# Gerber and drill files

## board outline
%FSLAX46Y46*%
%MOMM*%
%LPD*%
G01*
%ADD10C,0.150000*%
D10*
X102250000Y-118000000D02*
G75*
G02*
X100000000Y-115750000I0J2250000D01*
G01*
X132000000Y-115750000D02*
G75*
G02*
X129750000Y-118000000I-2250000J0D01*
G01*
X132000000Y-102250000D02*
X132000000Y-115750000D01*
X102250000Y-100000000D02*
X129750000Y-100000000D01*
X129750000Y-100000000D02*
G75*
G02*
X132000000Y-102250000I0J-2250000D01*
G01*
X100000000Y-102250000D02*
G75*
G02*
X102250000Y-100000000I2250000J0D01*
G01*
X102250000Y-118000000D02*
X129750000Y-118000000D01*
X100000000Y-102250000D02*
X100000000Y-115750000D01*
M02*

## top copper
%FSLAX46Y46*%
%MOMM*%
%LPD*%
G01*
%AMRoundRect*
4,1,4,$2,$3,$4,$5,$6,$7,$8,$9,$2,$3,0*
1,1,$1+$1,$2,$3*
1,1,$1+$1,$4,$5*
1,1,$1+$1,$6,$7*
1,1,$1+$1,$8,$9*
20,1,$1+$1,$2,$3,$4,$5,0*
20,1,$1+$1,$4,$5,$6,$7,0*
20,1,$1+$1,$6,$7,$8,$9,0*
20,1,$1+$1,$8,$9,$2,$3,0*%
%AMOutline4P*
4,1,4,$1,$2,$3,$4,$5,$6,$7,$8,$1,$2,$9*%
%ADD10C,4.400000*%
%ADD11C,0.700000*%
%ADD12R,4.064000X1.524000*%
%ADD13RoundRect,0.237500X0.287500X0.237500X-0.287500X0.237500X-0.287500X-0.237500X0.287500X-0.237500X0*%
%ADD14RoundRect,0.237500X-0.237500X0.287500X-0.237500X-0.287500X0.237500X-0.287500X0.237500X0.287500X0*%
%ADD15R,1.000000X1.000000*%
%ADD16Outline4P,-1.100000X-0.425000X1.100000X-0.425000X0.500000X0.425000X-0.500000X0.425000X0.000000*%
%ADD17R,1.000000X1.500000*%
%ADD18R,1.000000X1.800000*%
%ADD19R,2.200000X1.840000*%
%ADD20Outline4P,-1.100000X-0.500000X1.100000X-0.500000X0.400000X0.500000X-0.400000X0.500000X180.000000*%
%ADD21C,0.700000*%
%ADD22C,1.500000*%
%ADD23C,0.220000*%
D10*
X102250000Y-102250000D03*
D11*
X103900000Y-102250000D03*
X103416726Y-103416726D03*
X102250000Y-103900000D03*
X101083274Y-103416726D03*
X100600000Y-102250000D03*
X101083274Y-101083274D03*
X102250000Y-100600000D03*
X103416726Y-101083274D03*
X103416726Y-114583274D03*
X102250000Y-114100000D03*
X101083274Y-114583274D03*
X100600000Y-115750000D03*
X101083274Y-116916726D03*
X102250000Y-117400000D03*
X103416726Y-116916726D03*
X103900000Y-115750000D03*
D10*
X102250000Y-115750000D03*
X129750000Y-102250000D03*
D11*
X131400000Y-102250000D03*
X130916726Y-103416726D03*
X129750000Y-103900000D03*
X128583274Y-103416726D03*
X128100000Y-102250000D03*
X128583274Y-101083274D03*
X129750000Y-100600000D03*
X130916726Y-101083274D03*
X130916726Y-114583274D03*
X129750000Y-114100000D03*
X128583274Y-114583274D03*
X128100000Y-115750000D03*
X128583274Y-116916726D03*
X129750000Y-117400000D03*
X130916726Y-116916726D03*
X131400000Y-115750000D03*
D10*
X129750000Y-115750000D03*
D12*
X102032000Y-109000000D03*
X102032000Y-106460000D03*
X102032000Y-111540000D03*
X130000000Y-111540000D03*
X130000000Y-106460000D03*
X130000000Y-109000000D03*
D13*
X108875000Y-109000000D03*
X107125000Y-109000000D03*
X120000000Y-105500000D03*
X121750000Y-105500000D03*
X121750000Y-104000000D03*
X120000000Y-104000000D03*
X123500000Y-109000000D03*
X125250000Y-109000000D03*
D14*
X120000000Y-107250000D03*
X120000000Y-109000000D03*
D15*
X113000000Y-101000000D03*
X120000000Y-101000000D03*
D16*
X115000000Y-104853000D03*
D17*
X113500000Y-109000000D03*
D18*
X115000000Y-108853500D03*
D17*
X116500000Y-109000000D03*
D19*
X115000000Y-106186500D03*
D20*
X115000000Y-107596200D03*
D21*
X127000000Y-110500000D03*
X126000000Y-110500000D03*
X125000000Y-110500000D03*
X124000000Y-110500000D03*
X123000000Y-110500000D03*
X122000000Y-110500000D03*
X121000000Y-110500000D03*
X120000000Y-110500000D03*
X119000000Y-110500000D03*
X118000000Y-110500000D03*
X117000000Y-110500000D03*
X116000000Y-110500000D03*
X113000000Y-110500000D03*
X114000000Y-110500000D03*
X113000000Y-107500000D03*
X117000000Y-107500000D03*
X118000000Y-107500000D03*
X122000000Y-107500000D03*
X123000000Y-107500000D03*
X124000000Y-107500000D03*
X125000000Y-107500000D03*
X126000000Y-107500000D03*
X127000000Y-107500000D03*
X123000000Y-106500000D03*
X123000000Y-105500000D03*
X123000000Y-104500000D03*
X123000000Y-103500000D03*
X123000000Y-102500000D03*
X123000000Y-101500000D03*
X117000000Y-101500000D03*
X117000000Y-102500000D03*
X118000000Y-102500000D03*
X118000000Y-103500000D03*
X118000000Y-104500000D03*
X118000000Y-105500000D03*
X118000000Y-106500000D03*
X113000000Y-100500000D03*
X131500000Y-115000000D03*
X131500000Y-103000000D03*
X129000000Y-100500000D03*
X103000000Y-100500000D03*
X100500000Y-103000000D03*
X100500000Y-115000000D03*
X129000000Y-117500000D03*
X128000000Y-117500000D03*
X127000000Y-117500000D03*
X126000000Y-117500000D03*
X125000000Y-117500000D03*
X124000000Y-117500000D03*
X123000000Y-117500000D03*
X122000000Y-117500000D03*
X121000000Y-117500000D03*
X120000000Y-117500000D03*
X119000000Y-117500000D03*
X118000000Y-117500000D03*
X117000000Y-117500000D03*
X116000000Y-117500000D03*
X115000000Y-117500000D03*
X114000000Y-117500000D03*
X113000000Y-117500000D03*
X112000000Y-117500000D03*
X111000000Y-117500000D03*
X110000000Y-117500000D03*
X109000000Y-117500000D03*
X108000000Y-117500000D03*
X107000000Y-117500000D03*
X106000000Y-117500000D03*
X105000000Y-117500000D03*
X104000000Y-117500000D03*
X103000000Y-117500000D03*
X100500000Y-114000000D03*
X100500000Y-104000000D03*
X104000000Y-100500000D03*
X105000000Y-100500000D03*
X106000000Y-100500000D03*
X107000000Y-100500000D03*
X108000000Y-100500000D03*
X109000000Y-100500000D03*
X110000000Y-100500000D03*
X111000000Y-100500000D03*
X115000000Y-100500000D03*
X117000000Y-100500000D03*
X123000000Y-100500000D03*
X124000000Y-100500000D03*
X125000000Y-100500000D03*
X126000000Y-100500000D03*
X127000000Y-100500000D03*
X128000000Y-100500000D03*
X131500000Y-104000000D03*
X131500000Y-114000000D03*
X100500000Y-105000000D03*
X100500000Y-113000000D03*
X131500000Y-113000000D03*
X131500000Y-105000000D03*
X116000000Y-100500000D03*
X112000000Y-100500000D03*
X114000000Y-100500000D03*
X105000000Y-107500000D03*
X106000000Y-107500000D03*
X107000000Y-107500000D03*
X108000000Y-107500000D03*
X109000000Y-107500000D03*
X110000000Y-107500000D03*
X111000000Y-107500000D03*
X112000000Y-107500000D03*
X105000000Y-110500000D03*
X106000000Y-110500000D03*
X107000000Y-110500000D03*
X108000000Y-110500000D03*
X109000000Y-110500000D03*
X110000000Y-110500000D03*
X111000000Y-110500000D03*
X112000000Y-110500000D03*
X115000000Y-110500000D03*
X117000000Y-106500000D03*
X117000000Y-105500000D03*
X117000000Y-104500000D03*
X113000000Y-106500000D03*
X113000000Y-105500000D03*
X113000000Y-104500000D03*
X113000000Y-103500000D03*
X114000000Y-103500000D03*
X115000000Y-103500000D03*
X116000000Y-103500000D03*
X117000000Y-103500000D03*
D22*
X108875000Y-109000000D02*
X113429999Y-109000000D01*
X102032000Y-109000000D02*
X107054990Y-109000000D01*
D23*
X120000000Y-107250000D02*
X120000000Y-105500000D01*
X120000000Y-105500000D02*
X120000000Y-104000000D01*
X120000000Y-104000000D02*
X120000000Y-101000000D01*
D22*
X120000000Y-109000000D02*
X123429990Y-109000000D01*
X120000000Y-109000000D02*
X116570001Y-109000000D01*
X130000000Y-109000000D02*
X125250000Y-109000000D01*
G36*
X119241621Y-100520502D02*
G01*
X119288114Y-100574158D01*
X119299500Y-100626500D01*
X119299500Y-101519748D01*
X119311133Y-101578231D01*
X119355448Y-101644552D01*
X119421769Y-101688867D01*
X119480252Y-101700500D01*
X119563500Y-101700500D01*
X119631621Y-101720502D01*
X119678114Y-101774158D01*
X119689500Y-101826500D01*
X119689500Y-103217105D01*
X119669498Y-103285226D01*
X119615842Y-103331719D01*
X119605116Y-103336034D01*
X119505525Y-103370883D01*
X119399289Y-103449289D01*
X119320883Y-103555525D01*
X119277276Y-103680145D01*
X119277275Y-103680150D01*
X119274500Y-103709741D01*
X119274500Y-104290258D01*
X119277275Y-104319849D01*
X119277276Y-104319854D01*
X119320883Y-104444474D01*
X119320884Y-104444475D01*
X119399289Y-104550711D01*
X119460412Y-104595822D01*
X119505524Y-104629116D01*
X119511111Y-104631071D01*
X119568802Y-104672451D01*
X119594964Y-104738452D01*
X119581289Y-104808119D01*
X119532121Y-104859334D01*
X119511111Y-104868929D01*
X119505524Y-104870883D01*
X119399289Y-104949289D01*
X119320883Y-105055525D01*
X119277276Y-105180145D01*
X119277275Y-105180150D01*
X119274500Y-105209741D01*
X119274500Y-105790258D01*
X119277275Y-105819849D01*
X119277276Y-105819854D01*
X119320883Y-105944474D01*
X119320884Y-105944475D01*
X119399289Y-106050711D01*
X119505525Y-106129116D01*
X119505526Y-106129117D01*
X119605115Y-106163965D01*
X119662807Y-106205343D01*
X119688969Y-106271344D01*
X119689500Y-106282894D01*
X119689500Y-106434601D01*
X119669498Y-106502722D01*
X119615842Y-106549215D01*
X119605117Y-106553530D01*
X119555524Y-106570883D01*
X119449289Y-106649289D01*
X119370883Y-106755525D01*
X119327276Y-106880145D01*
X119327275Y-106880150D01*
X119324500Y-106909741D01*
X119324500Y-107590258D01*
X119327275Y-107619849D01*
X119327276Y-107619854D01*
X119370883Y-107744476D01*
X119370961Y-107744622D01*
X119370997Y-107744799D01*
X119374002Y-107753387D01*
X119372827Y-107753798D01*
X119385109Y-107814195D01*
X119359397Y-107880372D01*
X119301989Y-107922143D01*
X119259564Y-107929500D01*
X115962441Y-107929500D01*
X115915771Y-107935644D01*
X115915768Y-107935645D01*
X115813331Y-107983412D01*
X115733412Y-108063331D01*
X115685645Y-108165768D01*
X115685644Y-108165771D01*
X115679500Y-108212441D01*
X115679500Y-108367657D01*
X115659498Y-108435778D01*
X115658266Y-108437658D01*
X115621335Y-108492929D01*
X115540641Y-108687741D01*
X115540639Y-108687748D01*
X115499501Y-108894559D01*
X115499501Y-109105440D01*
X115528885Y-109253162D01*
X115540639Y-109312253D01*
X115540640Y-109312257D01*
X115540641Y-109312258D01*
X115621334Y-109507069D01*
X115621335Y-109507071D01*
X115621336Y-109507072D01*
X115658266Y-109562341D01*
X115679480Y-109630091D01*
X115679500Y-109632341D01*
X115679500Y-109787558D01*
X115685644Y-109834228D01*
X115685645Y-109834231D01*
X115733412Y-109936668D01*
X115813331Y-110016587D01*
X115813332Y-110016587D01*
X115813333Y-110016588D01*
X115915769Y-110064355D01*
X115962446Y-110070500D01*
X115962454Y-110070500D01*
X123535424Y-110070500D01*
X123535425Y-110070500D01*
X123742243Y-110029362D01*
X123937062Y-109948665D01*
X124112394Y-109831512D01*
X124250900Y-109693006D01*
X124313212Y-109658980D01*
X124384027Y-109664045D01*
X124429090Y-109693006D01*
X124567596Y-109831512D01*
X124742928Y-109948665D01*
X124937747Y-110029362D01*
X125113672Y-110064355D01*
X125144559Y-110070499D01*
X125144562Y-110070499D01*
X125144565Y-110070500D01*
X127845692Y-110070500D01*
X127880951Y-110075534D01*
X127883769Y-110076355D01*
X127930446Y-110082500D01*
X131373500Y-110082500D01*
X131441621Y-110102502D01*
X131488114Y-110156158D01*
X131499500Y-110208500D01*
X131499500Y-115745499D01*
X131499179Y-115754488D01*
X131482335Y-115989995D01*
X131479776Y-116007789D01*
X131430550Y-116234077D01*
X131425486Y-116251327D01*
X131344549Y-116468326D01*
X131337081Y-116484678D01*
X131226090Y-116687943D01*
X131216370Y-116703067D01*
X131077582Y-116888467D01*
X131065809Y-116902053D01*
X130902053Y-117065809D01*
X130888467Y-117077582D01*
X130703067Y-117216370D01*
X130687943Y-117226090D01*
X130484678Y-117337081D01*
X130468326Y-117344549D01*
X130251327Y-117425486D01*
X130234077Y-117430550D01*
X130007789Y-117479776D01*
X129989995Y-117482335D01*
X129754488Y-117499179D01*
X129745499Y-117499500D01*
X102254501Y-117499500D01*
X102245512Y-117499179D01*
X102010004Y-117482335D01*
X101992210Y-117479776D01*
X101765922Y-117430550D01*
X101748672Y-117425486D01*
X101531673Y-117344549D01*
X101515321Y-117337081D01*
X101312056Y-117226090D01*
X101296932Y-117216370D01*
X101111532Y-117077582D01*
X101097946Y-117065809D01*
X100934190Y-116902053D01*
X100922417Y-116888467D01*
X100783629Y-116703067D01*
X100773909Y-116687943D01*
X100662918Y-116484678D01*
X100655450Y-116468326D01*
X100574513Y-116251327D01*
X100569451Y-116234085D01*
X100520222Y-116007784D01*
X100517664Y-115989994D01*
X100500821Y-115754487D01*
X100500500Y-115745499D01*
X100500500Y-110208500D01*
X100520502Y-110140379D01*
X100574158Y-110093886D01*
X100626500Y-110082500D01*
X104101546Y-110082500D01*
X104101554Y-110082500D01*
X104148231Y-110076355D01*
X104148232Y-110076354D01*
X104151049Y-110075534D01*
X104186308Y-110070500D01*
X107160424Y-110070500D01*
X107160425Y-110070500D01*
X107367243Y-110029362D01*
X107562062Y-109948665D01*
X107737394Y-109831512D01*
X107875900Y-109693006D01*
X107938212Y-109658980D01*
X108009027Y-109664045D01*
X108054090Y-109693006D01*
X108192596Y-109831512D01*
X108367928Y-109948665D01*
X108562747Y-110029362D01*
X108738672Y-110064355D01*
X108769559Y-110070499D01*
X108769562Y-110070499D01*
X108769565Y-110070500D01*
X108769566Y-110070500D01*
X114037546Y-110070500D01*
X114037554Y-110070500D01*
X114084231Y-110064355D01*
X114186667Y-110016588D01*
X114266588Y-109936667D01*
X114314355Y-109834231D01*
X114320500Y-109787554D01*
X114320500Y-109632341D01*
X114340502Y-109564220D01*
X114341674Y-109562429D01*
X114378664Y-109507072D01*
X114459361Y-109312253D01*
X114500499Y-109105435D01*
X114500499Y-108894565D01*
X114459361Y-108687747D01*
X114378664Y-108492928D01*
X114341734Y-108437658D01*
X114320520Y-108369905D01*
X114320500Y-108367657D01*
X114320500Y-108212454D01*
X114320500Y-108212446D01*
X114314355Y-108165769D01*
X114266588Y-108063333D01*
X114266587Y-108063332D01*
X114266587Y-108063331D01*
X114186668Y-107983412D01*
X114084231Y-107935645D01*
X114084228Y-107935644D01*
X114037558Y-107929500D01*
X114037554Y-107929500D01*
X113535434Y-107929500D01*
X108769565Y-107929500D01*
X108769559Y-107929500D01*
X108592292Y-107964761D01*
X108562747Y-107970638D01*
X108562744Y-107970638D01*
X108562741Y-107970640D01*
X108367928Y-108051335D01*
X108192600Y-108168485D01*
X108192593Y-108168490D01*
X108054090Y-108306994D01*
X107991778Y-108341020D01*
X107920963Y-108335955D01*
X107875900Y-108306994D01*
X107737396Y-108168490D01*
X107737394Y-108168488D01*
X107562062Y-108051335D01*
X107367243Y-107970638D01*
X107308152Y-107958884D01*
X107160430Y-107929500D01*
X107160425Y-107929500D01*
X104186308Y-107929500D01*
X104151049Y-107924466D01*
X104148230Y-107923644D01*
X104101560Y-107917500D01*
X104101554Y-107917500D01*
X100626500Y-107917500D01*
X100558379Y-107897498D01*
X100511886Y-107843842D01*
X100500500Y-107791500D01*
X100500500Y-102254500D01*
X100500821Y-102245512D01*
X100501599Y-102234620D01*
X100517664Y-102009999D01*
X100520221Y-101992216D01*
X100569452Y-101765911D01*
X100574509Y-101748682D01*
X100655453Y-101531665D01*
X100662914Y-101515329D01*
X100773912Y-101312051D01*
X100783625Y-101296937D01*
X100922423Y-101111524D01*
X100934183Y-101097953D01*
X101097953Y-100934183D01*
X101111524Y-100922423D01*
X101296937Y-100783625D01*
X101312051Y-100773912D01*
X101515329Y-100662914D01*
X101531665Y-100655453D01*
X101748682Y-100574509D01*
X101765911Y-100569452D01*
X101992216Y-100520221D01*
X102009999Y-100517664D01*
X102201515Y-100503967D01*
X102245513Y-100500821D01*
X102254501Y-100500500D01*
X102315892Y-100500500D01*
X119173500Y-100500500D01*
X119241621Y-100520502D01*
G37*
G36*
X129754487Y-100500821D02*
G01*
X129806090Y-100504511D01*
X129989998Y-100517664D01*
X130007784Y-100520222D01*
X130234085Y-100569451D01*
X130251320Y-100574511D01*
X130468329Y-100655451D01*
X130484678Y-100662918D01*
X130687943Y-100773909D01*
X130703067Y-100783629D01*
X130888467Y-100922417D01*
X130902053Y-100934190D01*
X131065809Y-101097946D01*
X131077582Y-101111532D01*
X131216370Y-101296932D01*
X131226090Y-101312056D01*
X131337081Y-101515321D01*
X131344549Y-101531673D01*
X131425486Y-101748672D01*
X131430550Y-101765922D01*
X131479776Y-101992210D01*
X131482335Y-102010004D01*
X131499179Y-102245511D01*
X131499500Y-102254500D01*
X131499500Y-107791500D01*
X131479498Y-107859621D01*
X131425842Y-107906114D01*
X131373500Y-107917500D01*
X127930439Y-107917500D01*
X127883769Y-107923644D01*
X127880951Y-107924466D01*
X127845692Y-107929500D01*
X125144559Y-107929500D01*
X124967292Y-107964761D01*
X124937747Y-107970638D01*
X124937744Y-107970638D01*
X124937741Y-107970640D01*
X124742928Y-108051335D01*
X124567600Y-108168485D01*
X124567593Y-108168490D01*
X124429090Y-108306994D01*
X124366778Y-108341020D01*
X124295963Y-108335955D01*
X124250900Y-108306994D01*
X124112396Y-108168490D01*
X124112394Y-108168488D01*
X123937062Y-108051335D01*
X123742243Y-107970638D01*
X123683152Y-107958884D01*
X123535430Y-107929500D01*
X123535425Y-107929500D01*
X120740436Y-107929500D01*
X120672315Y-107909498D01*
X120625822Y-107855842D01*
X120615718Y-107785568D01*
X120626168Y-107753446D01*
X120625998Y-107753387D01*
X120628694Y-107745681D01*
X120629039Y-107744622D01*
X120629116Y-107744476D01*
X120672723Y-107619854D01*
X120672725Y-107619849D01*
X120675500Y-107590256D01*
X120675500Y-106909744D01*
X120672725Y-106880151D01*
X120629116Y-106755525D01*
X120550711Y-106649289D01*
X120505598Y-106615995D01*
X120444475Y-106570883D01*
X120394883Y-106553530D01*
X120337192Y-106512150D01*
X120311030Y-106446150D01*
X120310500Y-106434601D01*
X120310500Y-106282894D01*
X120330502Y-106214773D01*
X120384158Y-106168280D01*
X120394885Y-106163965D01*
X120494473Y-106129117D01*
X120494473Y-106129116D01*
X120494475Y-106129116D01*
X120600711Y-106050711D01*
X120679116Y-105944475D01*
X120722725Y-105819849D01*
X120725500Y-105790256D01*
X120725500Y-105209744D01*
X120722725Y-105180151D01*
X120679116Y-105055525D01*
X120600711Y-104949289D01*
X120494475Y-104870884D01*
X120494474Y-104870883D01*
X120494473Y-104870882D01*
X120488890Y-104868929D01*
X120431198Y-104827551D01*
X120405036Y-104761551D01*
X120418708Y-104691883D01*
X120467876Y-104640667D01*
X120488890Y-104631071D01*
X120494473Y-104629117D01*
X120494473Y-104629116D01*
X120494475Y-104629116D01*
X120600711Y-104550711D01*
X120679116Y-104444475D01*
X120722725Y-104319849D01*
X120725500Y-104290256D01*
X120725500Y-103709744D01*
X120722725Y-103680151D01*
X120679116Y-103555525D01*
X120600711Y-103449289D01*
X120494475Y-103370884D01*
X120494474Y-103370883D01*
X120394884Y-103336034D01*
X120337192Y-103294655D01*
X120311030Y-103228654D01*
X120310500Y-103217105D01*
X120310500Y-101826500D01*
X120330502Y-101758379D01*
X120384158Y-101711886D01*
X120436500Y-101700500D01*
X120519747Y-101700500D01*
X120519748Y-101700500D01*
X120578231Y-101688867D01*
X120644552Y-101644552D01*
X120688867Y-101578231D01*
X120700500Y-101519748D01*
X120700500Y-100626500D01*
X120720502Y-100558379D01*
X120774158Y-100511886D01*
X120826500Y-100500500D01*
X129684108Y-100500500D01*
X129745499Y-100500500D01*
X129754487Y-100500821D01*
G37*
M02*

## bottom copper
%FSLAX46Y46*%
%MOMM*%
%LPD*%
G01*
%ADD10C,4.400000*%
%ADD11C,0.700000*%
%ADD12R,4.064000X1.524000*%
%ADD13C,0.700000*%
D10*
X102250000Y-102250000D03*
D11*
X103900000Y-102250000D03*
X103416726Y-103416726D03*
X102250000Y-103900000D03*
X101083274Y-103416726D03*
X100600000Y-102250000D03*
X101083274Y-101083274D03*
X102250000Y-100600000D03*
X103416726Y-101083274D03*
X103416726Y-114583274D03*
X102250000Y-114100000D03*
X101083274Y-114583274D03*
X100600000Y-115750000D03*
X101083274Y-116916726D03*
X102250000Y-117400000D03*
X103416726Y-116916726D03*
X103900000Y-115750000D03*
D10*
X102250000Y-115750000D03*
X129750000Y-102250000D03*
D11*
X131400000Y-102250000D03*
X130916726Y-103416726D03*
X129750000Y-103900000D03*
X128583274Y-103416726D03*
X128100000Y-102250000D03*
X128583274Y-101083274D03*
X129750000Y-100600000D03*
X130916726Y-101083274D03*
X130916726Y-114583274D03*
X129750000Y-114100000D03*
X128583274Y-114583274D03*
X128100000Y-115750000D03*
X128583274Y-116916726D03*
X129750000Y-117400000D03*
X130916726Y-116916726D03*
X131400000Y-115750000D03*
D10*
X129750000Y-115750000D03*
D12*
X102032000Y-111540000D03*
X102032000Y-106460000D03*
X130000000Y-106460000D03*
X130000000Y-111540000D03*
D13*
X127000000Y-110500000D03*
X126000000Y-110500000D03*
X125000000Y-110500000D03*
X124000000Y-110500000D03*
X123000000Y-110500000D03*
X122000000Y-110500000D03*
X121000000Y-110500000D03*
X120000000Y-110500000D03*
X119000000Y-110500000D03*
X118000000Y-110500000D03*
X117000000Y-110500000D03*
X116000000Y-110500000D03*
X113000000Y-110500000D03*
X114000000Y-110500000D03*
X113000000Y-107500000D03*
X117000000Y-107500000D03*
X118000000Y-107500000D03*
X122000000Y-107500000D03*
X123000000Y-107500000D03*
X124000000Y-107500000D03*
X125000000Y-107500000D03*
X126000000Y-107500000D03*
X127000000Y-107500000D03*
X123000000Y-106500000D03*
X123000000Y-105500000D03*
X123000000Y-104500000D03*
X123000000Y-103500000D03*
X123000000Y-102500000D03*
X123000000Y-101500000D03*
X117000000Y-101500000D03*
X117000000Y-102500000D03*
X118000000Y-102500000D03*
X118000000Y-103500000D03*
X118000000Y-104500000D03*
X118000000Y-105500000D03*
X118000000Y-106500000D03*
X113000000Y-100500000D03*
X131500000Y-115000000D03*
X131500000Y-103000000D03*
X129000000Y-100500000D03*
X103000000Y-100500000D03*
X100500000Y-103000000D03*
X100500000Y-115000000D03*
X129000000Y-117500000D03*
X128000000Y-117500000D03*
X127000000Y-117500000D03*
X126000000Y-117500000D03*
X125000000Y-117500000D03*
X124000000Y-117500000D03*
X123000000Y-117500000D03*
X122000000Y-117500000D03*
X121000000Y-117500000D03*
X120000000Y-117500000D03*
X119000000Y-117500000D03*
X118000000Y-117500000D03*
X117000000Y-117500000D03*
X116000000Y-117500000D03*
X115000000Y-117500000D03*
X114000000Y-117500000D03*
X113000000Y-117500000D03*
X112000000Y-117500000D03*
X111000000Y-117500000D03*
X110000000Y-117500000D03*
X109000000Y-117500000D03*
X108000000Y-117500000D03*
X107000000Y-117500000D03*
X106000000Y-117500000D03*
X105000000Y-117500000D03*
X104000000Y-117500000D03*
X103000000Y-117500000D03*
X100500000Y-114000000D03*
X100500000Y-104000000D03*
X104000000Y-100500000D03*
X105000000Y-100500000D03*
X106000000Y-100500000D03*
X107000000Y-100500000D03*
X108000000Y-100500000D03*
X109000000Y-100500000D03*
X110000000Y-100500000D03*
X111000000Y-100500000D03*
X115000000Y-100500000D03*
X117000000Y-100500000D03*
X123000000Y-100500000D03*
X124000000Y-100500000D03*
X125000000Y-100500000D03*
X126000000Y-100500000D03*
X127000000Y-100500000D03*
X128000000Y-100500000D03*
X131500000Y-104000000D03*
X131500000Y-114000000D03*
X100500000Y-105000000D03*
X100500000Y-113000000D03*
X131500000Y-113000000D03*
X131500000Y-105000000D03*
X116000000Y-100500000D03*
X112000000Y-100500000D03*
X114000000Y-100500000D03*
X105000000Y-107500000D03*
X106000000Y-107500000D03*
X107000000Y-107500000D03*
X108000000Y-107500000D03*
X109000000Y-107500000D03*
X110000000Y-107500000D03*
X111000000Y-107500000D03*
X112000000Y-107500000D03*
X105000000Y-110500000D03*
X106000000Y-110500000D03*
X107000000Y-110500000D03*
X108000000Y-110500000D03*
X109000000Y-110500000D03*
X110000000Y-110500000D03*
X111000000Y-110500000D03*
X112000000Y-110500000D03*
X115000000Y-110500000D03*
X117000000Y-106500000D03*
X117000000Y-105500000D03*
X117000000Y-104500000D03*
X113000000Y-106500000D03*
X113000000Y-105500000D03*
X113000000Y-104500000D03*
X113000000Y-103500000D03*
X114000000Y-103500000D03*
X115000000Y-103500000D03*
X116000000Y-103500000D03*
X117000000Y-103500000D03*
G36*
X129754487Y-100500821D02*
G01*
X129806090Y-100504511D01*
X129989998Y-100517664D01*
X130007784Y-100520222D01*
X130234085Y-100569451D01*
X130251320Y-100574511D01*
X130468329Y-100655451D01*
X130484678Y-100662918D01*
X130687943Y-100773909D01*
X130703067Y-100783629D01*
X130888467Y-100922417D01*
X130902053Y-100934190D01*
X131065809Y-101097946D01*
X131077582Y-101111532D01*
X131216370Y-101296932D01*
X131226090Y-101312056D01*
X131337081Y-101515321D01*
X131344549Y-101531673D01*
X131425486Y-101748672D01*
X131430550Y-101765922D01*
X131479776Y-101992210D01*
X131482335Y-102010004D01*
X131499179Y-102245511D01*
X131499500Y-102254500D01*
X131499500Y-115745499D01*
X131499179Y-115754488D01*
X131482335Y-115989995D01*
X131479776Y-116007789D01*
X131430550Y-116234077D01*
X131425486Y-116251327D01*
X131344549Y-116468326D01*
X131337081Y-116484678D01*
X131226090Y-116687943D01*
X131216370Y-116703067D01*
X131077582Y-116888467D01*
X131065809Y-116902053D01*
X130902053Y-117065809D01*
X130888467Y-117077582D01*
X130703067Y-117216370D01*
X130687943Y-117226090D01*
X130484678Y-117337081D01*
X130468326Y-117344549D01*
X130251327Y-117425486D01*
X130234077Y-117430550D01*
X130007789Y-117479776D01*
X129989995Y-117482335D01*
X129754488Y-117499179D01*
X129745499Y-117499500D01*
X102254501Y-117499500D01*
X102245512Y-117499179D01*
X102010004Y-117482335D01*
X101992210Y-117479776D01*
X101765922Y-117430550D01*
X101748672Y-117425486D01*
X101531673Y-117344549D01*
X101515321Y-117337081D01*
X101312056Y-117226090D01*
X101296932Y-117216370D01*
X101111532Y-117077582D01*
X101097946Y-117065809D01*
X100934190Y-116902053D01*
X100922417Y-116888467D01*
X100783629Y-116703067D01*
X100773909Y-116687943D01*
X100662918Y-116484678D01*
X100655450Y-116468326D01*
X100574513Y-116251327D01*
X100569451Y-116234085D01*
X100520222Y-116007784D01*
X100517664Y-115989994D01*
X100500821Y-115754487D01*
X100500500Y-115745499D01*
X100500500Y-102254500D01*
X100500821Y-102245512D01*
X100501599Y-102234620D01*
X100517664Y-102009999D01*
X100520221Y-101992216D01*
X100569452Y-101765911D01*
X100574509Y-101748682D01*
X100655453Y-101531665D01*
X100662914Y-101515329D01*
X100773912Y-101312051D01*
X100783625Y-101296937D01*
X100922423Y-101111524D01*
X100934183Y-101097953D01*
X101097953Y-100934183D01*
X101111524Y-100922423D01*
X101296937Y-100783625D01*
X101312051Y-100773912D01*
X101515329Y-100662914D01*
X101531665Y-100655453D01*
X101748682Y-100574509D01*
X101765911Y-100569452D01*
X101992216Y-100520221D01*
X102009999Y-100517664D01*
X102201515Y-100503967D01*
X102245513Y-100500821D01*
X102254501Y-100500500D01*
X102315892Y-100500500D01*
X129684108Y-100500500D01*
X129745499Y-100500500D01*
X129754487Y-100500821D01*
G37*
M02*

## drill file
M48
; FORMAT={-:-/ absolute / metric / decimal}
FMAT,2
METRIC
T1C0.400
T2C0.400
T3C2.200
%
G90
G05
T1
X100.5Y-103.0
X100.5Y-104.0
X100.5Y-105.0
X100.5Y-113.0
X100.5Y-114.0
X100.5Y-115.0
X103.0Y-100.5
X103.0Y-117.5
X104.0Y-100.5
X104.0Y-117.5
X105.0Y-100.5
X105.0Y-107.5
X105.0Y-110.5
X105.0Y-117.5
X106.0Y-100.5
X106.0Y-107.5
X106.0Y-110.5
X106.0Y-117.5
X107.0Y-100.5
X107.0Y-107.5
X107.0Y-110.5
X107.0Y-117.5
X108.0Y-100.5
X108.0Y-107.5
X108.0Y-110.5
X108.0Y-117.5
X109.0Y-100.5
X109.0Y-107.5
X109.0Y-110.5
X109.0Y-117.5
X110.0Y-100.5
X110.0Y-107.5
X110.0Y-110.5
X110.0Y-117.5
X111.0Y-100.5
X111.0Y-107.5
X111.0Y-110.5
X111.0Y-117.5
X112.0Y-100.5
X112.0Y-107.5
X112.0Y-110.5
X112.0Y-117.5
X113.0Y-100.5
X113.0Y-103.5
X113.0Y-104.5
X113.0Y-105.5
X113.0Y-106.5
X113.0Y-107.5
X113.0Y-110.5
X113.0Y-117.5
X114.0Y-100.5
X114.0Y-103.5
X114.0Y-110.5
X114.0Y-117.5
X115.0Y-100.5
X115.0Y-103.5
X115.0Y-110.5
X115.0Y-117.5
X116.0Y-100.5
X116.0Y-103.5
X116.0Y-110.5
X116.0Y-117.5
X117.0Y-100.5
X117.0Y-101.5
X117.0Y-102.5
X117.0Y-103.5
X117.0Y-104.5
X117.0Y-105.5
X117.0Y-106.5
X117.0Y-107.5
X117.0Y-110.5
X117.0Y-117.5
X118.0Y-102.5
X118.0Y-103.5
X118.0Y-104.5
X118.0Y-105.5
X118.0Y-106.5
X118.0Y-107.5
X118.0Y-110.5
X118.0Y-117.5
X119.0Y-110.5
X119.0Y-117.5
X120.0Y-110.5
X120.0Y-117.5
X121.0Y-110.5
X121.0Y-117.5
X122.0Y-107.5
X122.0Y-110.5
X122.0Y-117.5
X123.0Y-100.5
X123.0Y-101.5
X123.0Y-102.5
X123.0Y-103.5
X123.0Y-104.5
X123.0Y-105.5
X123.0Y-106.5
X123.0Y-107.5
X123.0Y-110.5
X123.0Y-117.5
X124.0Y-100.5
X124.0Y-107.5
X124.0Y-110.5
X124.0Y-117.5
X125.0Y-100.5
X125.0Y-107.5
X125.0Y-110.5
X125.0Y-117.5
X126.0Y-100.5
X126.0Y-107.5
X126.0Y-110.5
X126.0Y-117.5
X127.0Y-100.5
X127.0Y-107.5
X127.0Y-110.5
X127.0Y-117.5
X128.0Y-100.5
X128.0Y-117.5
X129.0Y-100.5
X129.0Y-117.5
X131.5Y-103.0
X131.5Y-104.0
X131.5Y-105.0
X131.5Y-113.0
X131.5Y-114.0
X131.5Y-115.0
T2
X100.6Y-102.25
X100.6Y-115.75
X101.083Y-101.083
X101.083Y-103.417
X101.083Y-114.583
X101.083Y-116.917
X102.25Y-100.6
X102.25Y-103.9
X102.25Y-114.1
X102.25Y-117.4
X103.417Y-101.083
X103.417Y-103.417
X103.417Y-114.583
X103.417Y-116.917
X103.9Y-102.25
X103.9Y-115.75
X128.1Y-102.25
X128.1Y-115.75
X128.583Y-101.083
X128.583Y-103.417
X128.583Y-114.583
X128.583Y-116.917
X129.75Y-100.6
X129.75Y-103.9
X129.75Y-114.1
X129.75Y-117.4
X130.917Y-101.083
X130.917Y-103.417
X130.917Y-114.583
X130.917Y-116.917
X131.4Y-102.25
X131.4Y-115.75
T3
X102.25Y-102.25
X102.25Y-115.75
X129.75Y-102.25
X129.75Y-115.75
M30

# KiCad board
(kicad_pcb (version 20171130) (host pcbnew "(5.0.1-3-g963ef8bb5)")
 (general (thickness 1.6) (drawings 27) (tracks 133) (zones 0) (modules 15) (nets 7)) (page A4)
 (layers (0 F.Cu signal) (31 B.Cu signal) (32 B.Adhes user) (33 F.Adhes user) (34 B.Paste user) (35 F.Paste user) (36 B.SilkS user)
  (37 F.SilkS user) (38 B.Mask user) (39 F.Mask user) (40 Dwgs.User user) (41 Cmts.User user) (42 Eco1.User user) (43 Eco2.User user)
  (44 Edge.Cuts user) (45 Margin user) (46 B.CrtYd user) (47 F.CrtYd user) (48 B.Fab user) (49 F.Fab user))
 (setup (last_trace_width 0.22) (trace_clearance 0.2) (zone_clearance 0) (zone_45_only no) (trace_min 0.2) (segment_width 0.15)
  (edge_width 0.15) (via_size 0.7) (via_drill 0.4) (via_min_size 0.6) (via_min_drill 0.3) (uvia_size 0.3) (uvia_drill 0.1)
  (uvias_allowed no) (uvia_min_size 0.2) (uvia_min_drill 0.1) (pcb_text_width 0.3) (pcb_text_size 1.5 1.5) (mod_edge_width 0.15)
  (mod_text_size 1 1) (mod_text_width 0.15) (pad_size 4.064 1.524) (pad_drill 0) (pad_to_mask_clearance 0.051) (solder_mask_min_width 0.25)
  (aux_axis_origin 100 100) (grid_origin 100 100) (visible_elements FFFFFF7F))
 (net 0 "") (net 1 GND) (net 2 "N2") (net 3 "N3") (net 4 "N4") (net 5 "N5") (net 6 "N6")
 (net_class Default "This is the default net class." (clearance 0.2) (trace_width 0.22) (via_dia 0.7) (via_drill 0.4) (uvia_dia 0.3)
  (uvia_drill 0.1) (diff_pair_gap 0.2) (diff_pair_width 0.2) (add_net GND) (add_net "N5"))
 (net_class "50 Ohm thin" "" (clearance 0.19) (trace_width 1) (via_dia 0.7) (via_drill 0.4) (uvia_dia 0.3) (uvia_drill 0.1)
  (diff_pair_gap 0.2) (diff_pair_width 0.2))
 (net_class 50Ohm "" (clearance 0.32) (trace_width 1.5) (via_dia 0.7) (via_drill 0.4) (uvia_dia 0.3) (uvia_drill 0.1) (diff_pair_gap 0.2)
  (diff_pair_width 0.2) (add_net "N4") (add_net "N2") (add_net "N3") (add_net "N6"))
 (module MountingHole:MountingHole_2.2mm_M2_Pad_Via (layer F.Cu) (at 102.25 102.25)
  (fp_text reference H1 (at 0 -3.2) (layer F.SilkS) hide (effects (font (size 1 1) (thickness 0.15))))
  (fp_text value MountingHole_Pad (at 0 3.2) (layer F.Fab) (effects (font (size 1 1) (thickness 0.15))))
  (pad 1 thru_hole circle (at 0 0) (size 4.4 4.4) (drill 2.2) (layers *.Cu *.Mask) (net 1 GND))
  (pad 1 thru_hole circle (at 1.65 0) (size 0.7 0.7) (drill 0.4) (layers *.Cu *.Mask) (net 1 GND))
  (pad 1 thru_hole circle (at 1.166726 1.166726) (size 0.7 0.7) (drill 0.4) (layers *.Cu *.Mask) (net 1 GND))
  (pad 1 thru_hole circle (at 0 1.65) (size 0.7 0.7) (drill 0.4) (layers *.Cu *.Mask) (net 1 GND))
  (pad 1 thru_hole circle (at -1.166726 1.166726) (size 0.7 0.7) (drill 0.4) (layers *.Cu *.Mask) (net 1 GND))
  (pad 1 thru_hole circle (at -1.65 0) (size 0.7 0.7) (drill 0.4) (layers *.Cu *.Mask) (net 1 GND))
  (pad 1 thru_hole circle (at -1.166726 -1.166726) (size 0.7 0.7) (drill 0.4) (layers *.Cu *.Mask) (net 1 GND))
  (pad 1 thru_hole circle (at 0 -1.65) (size 0.7 0.7) (drill 0.4) (layers *.Cu *.Mask) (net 1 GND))
  (pad 1 thru_hole circle (at 1.166726 -1.166726) (size 0.7 0.7) (drill 0.4) (layers *.Cu *.Mask) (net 1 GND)))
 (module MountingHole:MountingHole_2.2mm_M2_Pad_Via (layer F.Cu) (at 102.25 115.75)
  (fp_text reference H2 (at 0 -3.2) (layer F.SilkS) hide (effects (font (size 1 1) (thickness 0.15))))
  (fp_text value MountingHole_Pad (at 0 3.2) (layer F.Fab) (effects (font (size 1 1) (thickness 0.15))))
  (pad 1 thru_hole circle (at 1.166726 -1.166726) (size 0.7 0.7) (drill 0.4) (layers *.Cu *.Mask) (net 1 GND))
  (pad 1 thru_hole circle (at 0 -1.65) (size 0.7 0.7) (drill 0.4) (layers *.Cu *.Mask) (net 1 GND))
  (pad 1 thru_hole circle (at -1.166726 -1.166726) (size 0.7 0.7) (drill 0.4) (layers *.Cu *.Mask) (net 1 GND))
  (pad 1 thru_hole circle (at -1.65 0) (size 0.7 0.7) (drill 0.4) (layers *.Cu *.Mask) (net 1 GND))
  (pad 1 thru_hole circle (at -1.166726 1.166726) (size 0.7 0.7) (drill 0.4) (layers *.Cu *.Mask) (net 1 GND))
  (pad 1 thru_hole circle (at 0 1.65) (size 0.7 0.7) (drill 0.4) (layers *.Cu *.Mask) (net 1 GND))
  (pad 1 thru_hole circle (at 1.166726 1.166726) (size 0.7 0.7) (drill 0.4) (layers *.Cu *.Mask) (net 1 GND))
  (pad 1 thru_hole circle (at 1.65 0) (size 0.7 0.7) (drill 0.4) (layers *.Cu *.Mask) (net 1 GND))
  (pad 1 thru_hole circle (at 0 0) (size 4.4 4.4) (drill 2.2) (layers *.Cu *.Mask) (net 1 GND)))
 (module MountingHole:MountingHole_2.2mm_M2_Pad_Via (layer F.Cu) (at 129.75 102.25)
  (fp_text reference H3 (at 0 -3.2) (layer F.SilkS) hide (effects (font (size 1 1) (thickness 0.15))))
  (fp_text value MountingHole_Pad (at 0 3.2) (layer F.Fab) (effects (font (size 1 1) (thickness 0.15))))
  (pad 1 thru_hole circle (at 0 0) (size 4.4 4.4) (drill 2.2) (layers *.Cu *.Mask) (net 1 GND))
  (pad 1 thru_hole circle (at 1.65 0) (size 0.7 0.7) (drill 0.4) (layers *.Cu *.Mask) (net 1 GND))
  (pad 1 thru_hole circle (at 1.166726 1.166726) (size 0.7 0.7) (drill 0.4) (layers *.Cu *.Mask) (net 1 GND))
  (pad 1 thru_hole circle (at 0 1.65) (size 0.7 0.7) (drill 0.4) (layers *.Cu *.Mask) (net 1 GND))
  (pad 1 thru_hole circle (at -1.166726 1.166726) (size 0.7 0.7) (drill 0.4) (layers *.Cu *.Mask) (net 1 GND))
  (pad 1 thru_hole circle (at -1.65 0) (size 0.7 0.7) (drill 0.4) (layers *.Cu *.Mask) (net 1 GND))
  (pad 1 thru_hole circle (at -1.166726 -1.166726) (size 0.7 0.7) (drill 0.4) (layers *.Cu *.Mask) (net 1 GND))
  (pad 1 thru_hole circle (at 0 -1.65) (size 0.7 0.7) (drill 0.4) (layers *.Cu *.Mask) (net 1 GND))
  (pad 1 thru_hole circle (at 1.166726 -1.166726) (size 0.7 0.7) (drill 0.4) (layers *.Cu *.Mask) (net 1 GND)))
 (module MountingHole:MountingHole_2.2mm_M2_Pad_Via (layer F.Cu) (at 129.75 115.75)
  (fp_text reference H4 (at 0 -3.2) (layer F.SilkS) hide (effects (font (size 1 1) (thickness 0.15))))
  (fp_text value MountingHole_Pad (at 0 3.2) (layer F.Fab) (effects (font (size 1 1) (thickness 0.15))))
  (pad 1 thru_hole circle (at 1.166726 -1.166726) (size 0.7 0.7) (drill 0.4) (layers *.Cu *.Mask) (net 1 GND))
  (pad 1 thru_hole circle (at 0 -1.65) (size 0.7 0.7) (drill 0.4) (layers *.Cu *.Mask) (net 1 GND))
  (pad 1 thru_hole circle (at -1.166726 -1.166726) (size 0.7 0.7) (drill 0.4) (layers *.Cu *.Mask) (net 1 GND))
  (pad 1 thru_hole circle (at -1.65 0) (size 0.7 0.7) (drill 0.4) (layers *.Cu *.Mask) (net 1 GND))
  (pad 1 thru_hole circle (at -1.166726 1.166726) (size 0.7 0.7) (drill 0.4) (layers *.Cu *.Mask) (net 1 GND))
  (pad 1 thru_hole circle (at 0 1.65) (size 0.7 0.7) (drill 0.4) (layers *.Cu *.Mask) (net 1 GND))
  (pad 1 thru_hole circle (at 1.166726 1.166726) (size 0.7 0.7) (drill 0.4) (layers *.Cu *.Mask) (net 1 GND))
  (pad 1 thru_hole circle (at 1.65 0) (size 0.7 0.7) (drill 0.4) (layers *.Cu *.Mask) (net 1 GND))
  (pad 1 thru_hole circle (at 0 0) (size 4.4 4.4) (drill 2.2) (layers *.Cu *.Mask) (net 1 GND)))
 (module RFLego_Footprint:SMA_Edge (layer F.Cu) (at 100 109)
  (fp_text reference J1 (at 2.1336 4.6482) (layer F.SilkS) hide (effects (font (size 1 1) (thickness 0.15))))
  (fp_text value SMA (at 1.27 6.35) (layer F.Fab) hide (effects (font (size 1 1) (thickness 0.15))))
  (pad 1 smd rect (at 2.032 0) (size 4.064 1.524) (layers F.Cu F.Mask) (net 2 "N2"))
  (pad 2 smd rect (at 2.032 -2.54) (size 4.064 1.524) (layers F.Cu F.Mask) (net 1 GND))
  (pad 2 smd rect (at 2.032 2.54) (size 4.064 1.524) (layers B.Cu B.Mask) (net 1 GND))
  (pad 2 smd rect (at 2.032 -2.54) (size 4.064 1.524) (layers B.Cu B.Mask) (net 1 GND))
  (pad 2 smd rect (at 2.032 2.54) (size 4.064 1.524) (layers F.Cu F.Mask) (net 1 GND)))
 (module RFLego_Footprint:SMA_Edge (layer F.Cu) (at 127.968 109)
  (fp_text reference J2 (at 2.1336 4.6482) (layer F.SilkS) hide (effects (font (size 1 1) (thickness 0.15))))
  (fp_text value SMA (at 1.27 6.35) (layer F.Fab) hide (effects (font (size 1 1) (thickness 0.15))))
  (pad 2 smd rect (at 2.032 2.54) (size 4.064 1.524) (layers F.Cu F.Mask) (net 1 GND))
  (pad 2 smd rect (at 2.032 -2.54) (size 4.064 1.524) (layers B.Cu B.Mask) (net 1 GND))
  (pad 2 smd rect (at 2.032 2.54) (size 4.064 1.524) (layers B.Cu B.Mask) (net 1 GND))
  (pad 2 smd rect (at 2.032 -2.54) (size 4.064 1.524) (layers F.Cu F.Mask) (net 1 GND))
  (pad 1 smd rect (at 2.032 0) (size 4.064 1.524) (layers F.Cu F.Mask) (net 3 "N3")))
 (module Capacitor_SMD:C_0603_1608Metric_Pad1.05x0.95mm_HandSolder (layer F.Cu) (at 108 109 180)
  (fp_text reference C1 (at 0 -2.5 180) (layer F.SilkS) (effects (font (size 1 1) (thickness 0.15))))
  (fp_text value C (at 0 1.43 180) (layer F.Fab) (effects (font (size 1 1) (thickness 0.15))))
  (pad 1 smd roundrect (at -0.875 0 180) (size 1.05 0.95) (layers F.Cu F.Paste F.Mask) (roundrect_rratio 0.25) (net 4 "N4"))
  (pad 2 smd roundrect (at 0.875 0 180) (size 1.05 0.95) (layers F.Cu F.Paste F.Mask) (roundrect_rratio 0.25) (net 2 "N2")))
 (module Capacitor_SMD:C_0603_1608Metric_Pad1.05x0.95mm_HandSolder (layer F.Cu) (at 120.875 105.5 180)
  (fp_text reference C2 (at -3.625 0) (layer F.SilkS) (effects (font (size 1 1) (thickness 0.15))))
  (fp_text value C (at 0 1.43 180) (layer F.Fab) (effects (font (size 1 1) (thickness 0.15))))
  (pad 2 smd roundrect (at 0.875 0 180) (size 1.05 0.95) (layers F.Cu F.Paste F.Mask) (roundrect_rratio 0.25) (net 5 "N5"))
  (pad 1 smd roundrect (at -0.875 0 180) (size 1.05 0.95) (layers F.Cu F.Paste F.Mask) (roundrect_rratio 0.25) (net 1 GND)))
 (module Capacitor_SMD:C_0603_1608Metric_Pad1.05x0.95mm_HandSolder (layer F.Cu) (at 120.875 104 180)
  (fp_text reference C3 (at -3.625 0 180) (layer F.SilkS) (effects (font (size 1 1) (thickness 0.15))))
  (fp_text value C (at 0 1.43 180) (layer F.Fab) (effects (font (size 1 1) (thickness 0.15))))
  (pad 1 smd roundrect (at -0.875 0 180) (size 1.05 0.95) (layers F.Cu F.Paste F.Mask) (roundrect_rratio 0.25) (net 1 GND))
  (pad 2 smd roundrect (at 0.875 0 180) (size 1.05 0.95) (layers F.Cu F.Paste F.Mask) (roundrect_rratio 0.25) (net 5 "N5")))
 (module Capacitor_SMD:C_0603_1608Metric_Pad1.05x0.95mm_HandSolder (layer F.Cu) (at 124.375 109 180)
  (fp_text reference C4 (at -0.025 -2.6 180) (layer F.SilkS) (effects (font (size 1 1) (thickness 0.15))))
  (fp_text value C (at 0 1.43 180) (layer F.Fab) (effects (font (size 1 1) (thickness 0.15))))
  (pad 2 smd roundrect (at 0.875 0 180) (size 1.05 0.95) (layers F.Cu F.Paste F.Mask) (roundrect_rratio 0.25) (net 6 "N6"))
  (pad 1 smd roundrect (at -0.875 0 180) (size 1.05 0.95) (layers F.Cu F.Paste F.Mask) (roundrect_rratio 0.25) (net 3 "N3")))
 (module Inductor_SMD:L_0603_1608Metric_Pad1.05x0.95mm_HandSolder (layer F.Cu) (at 120 108.125 270)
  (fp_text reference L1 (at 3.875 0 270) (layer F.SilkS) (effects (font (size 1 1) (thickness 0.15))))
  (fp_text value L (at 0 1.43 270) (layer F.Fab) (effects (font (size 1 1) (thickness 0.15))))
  (pad 1 smd roundrect (at -0.875 0 270) (size 1.05 0.95) (layers F.Cu F.Paste F.Mask) (roundrect_rratio 0.25) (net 5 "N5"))
  (pad 2 smd roundrect (at 0.875 0 270) (size 1.05 0.95) (layers F.Cu F.Paste F.Mask) (roundrect_rratio 0.25) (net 6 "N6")))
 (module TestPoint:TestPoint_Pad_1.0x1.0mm (layer F.Cu) (at 113 101)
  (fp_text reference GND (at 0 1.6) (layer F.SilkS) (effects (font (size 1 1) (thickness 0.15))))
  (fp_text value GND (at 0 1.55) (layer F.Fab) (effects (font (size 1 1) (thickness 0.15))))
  (pad 1 smd rect (at 0 0) (size 1 1) (layers F.Cu F.Mask) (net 1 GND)))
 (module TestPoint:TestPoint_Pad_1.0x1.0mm (layer F.Cu) (at 120 101)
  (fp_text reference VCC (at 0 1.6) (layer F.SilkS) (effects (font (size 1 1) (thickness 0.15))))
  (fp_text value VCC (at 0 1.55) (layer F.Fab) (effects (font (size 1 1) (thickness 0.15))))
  (pad 1 smd rect (at 0 0) (size 1 1) (layers F.Cu F.Mask) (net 5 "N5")))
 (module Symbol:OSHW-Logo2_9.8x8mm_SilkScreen (layer B.Cu) (at 109.5 113 180)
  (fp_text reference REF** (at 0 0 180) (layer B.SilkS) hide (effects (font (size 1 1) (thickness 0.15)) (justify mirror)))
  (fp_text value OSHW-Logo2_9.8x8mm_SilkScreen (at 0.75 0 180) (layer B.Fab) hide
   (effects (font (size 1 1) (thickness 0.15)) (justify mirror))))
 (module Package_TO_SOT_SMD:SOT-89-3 (layer F.Cu) (at 115 107.52 90)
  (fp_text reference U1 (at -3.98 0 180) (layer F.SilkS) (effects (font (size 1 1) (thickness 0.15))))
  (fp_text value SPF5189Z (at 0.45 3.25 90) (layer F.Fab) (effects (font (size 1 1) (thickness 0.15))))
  (pad 2 smd trapezoid (at 2.667 0) (size 1.6 0.85) (rect_delta 0 0.6) (layers F.Cu F.Paste F.Mask) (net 1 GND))
  (pad 1 smd rect (at -1.48 -1.5) (size 1 1.5) (layers F.Cu F.Paste F.Mask) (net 4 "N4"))
  (pad 2 smd rect (at -1.3335 0) (size 1 1.8) (layers F.Cu F.Paste F.Mask) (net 1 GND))
  (pad 3 smd rect (at -1.48 1.5) (size 1 1.5) (layers F.Cu F.Paste F.Mask) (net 6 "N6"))
  (pad 2 smd rect (at 1.3335 0) (size 2.2 1.84) (layers F.Cu F.Paste F.Mask) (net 1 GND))
  (pad 2 smd trapezoid (at -0.0762 0 180) (size 1.5 1) (rect_delta 0 0.7) (layers F.Cu F.Paste F.Mask) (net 1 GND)))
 (gr_arc (start 102.25 115.75) (end 100 115.75) (angle -90) (layer Edge.Cuts) (width 0.15))
 (gr_arc (start 129.75 115.75) (end 129.75 118) (angle -90) (layer Edge.Cuts) (width 0.15))
 (gr_line (start 132 102.25) (end 132 115.75) (layer Edge.Cuts) (width 0.15))
 (gr_line (start 102.25 100) (end 129.75 100) (layer Edge.Cuts) (width 0.15))
 (gr_arc (start 129.75 102.25) (end 132 102.25) (angle -90) (layer Edge.Cuts) (width 0.15))
 (gr_arc (start 102.25 102.25) (end 102.25 100) (angle -90) (layer Edge.Cuts) (width 0.15))
 (gr_line (start 102.25 118) (end 129.75 118) (layer Edge.Cuts) (width 0.15))
 (gr_line (start 100 102.25) (end 100 115.75) (layer Edge.Cuts) (width 0.15))
 (via (at 127 110.5) (size 0.7) (drill 0.4) (layers F.Cu B.Cu) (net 1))
 (via (at 126 110.5) (size 0.7) (drill 0.4) (layers F.Cu B.Cu) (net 1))
 (via (at 125 110.5) (size 0.7) (drill 0.4) (layers F.Cu B.Cu) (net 1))
 (via (at 124 110.5) (size 0.7) (drill 0.4) (layers F.Cu B.Cu) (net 1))
 (via (at 123 110.5) (size 0.7) (drill 0.4) (layers F.Cu B.Cu) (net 1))
 (via (at 122 110.5) (size 0.7) (drill 0.4) (layers F.Cu B.Cu) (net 1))
 (via (at 121 110.5) (size 0.7) (drill 0.4) (layers F.Cu B.Cu) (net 1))
 (via (at 120 110.5) (size 0.7) (drill 0.4) (layers F.Cu B.Cu) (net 1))
 (via (at 119 110.5) (size 0.7) (drill 0.4) (layers F.Cu B.Cu) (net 1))
 (via (at 118 110.5) (size 0.7) (drill 0.4) (layers F.Cu B.Cu) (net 1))
 (via (at 117 110.5) (size 0.7) (drill 0.4) (layers F.Cu B.Cu) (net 1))
 (via (at 116 110.5) (size 0.7) (drill 0.4) (layers F.Cu B.Cu) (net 1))
 (via (at 113 110.5) (size 0.7) (drill 0.4) (layers F.Cu B.Cu) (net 1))
 (via (at 114 110.5) (size 0.7) (drill 0.4) (layers F.Cu B.Cu) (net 1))
 (via (at 113 107.5) (size 0.7) (drill 0.4) (layers F.Cu B.Cu) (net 1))
 (via (at 117 107.5) (size 0.7) (drill 0.4) (layers F.Cu B.Cu) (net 1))
 (via (at 118 107.5) (size 0.7) (drill 0.4) (layers F.Cu B.Cu) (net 1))
 (via (at 122 107.5) (size 0.7) (drill 0.4) (layers F.Cu B.Cu) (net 1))
 (via (at 123 107.5) (size 0.7) (drill 0.4) (layers F.Cu B.Cu) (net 1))
 (via (at 124 107.5) (size 0.7) (drill 0.4) (layers F.Cu B.Cu) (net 1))
 (via (at 125 107.5) (size 0.7) (drill 0.4) (layers F.Cu B.Cu) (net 1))
 (via (at 126 107.5) (size 0.7) (drill 0.4) (layers F.Cu B.Cu) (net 1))
 (via (at 127 107.5) (size 0.7) (drill 0.4) (layers F.Cu B.Cu) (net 1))
 (via (at 123 106.5) (size 0.7) (drill 0.4) (layers F.Cu B.Cu) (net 1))
 (via (at 123 105.5) (size 0.7) (drill 0.4) (layers F.Cu B.Cu) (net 1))
 (via (at 123 104.5) (size 0.7) (drill 0.4) (layers F.Cu B.Cu) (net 1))
 (via (at 123 103.5) (size 0.7) (drill 0.4) (layers F.Cu B.Cu) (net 1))
 (via (at 123 102.5) (size 0.7) (drill 0.4) (layers F.Cu B.Cu) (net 1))
 (via (at 123 101.5) (size 0.7) (drill 0.4) (layers F.Cu B.Cu) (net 1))
 (via (at 117 101.5) (size 0.7) (drill 0.4) (layers F.Cu B.Cu) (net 1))
 (via (at 117 102.5) (size 0.7) (drill 0.4) (layers F.Cu B.Cu) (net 1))
 (via (at 118 102.5) (size 0.7) (drill 0.4) (layers F.Cu B.Cu) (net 1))
 (via (at 118 103.5) (size 0.7) (drill 0.4) (layers F.Cu B.Cu) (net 1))
 (via (at 118 104.5) (size 0.7) (drill 0.4) (layers F.Cu B.Cu) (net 1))
 (via (at 118 105.5) (size 0.7) (drill 0.4) (layers F.Cu B.Cu) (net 1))
 (via (at 118 106.5) (size 0.7) (drill 0.4) (layers F.Cu B.Cu) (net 1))
 (via (at 113 100.5) (size 0.7) (drill 0.4) (layers F.Cu B.Cu) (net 1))
 (via (at 131.5 115) (size 0.7) (drill 0.4) (layers F.Cu B.Cu) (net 1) (status 30))
 (via (at 131.5 103) (size 0.7) (drill 0.4) (layers F.Cu B.Cu) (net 1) (status 30))
 (via (at 129 100.5) (size 0.7) (drill 0.4) (layers F.Cu B.Cu) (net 1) (status 30))
 (via (at 103 100.5) (size 0.7) (drill 0.4) (layers F.Cu B.Cu) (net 1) (status 30))
 (via (at 100.5 103) (size 0.7) (drill 0.4) (layers F.Cu B.Cu) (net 1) (status 30))
 (via (at 100.5 115) (size 0.7) (drill 0.4) (layers F.Cu B.Cu) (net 1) (status 30))
 (via (at 129 117.5) (size 0.7) (drill 0.4) (layers F.Cu B.Cu) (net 1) (status 30))
 (via (at 128 117.5) (size 0.7) (drill 0.4) (layers F.Cu B.Cu) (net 1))
 (via (at 127 117.5) (size 0.7) (drill 0.4) (layers F.Cu B.Cu) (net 1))
 (via (at 126 117.5) (size 0.7) (drill 0.4) (layers F.Cu B.Cu) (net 1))
 (via (at 125 117.5) (size 0.7) (drill 0.4) (layers F.Cu B.Cu) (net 1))
 (via (at 124 117.5) (size 0.7) (drill 0.4) (layers F.Cu B.Cu) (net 1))
 (via (at 123 117.5) (size 0.7) (drill 0.4) (layers F.Cu B.Cu) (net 1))
 (via (at 122 117.5) (size 0.7) (drill 0.4) (layers F.Cu B.Cu) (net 1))
 (via (at 121 117.5) (size 0.7) (drill 0.4) (layers F.Cu B.Cu) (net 1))
 (via (at 120 117.5) (size 0.7) (drill 0.4) (layers F.Cu B.Cu) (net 1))
 (via (at 119 117.5) (size 0.7) (drill 0.4) (layers F.Cu B.Cu) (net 1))
 (via (at 118 117.5) (size 0.7) (drill 0.4) (layers F.Cu B.Cu) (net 1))
 (via (at 117 117.5) (size 0.7) (drill 0.4) (layers F.Cu B.Cu) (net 1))
 (via (at 116 117.5) (size 0.7) (drill 0.4) (layers F.Cu B.Cu) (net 1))
 (via (at 115 117.5) (size 0.7) (drill 0.4) (layers F.Cu B.Cu) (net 1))
 (via (at 114 117.5) (size 0.7) (drill 0.4) (layers F.Cu B.Cu) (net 1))
 (via (at 113 117.5) (size 0.7) (drill 0.4) (layers F.Cu B.Cu) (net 1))
 (via (at 112 117.5) (size 0.7) (drill 0.4) (layers F.Cu B.Cu) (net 1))
 (via (at 111 117.5) (size 0.7) (drill 0.4) (layers F.Cu B.Cu) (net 1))
 (via (at 110 117.5) (size 0.7) (drill 0.4) (layers F.Cu B.Cu) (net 1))
 (via (at 109 117.5) (size 0.7) (drill 0.4) (layers F.Cu B.Cu) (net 1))
 (via (at 108 117.5) (size 0.7) (drill 0.4) (layers F.Cu B.Cu) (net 1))
 (via (at 107 117.5) (size 0.7) (drill 0.4) (layers F.Cu B.Cu) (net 1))
 (via (at 106 117.5) (size 0.7) (drill 0.4) (layers F.Cu B.Cu) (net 1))
 (via (at 105 117.5) (size 0.7) (drill 0.4) (layers F.Cu B.Cu) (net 1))
 (via (at 104 117.5) (size 0.7) (drill 0.4) (layers F.Cu B.Cu) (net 1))
 (via (at 103 117.5) (size 0.7) (drill 0.4) (layers F.Cu B.Cu) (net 1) (status 30))
 (via (at 100.5 114) (size 0.7) (drill 0.4) (layers F.Cu B.Cu) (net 1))
 (via (at 100.5 104) (size 0.7) (drill 0.4) (layers F.Cu B.Cu) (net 1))
 (via (at 104 100.5) (size 0.7) (drill 0.4) (layers F.Cu B.Cu) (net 1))
 (via (at 105 100.5) (size 0.7) (drill 0.4) (layers F.Cu B.Cu) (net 1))
 (via (at 106 100.5) (size 0.7) (drill 0.4) (layers F.Cu B.Cu) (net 1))
 (via (at 107 100.5) (size 0.7) (drill 0.4) (layers F.Cu B.Cu) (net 1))
 (via (at 108 100.5) (size 0.7) (drill 0.4) (layers F.Cu B.Cu) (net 1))
 (via (at 109 100.5) (size 0.7) (drill 0.4) (layers F.Cu B.Cu) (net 1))
 (via (at 110 100.5) (size 0.7) (drill 0.4) (layers F.Cu B.Cu) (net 1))
 (via (at 111 100.5) (size 0.7) (drill 0.4) (layers F.Cu B.Cu) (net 1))
 (via (at 115 100.5) (size 0.7) (drill 0.4) (layers F.Cu B.Cu) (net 1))
 (via (at 117 100.5) (size 0.7) (drill 0.4) (layers F.Cu B.Cu) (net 1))
 (via (at 123 100.5) (size 0.7) (drill 0.4) (layers F.Cu B.Cu) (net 1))
 (via (at 124 100.5) (size 0.7) (drill 0.4) (layers F.Cu B.Cu) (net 1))
 (via (at 125 100.5) (size 0.7) (drill 0.4) (layers F.Cu B.Cu) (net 1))
 (via (at 126 100.5) (size 0.7) (drill 0.4) (layers F.Cu B.Cu) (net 1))
 (via (at 127 100.5) (size 0.7) (drill 0.4) (layers F.Cu B.Cu) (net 1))
 (via (at 128 100.5) (size 0.7) (drill 0.4) (layers F.Cu B.Cu) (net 1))
 (via (at 131.5 104) (size 0.7) (drill 0.4) (layers F.Cu B.Cu) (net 1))
 (via (at 131.5 114) (size 0.7) (drill 0.4) (layers F.Cu B.Cu) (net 1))
 (via (at 100.5 105) (size 0.7) (drill 0.4) (layers F.Cu B.Cu) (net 1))
 (via (at 100.5 113) (size 0.7) (drill 0.4) (layers F.Cu B.Cu) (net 1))
 (via (at 131.5 113) (size 0.7) (drill 0.4) (layers F.Cu B.Cu) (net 1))
 (via (at 131.5 105) (size 0.7) (drill 0.4) (layers F.Cu B.Cu) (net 1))
 (via (at 116 100.5) (size 0.7) (drill 0.4) (layers F.Cu B.Cu) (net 1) (status 30))
 (via (at 112 100.5) (size 0.7) (drill 0.4) (layers F.Cu B.Cu) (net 1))
 (via (at 114 100.5) (size 0.7) (drill 0.4) (layers F.Cu B.Cu) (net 1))
 (via (at 105 107.5) (size 0.7) (drill 0.4) (layers F.Cu B.Cu) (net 1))
 (via (at 106 107.5) (size 0.7) (drill 0.4) (layers F.Cu B.Cu) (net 1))
 (via (at 107 107.5) (size 0.7) (drill 0.4) (layers F.Cu B.Cu) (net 1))
 (via (at 108 107.5) (size 0.7) (drill 0.4) (layers F.Cu B.Cu) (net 1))
 (via (at 109 107.5) (size 0.7) (drill 0.4) (layers F.Cu B.Cu) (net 1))
 (via (at 110 107.5) (size 0.7) (drill 0.4) (layers F.Cu B.Cu) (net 1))
 (via (at 111 107.5) (size 0.7) (drill 0.4) (layers F.Cu B.Cu) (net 1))
 (via (at 112 107.5) (size 0.7) (drill 0.4) (layers F.Cu B.Cu) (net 1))
 (via (at 105 110.5) (size 0.7) (drill 0.4) (layers F.Cu B.Cu) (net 1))
 (via (at 106 110.5) (size 0.7) (drill 0.4) (layers F.Cu B.Cu) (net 1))
 (via (at 107 110.5) (size 0.7) (drill 0.4) (layers F.Cu B.Cu) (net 1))
 (via (at 108 110.5) (size 0.7) (drill 0.4) (layers F.Cu B.Cu) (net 1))
 (via (at 109 110.5) (size 0.7) (drill 0.4) (layers F.Cu B.Cu) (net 1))
 (via (at 110 110.5) (size 0.7) (drill 0.4) (layers F.Cu B.Cu) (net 1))
 (via (at 111 110.5) (size 0.7) (drill 0.4) (layers F.Cu B.Cu) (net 1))
 (via (at 112 110.5) (size 0.7) (drill 0.4) (layers F.Cu B.Cu) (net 1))
 (via (at 115 110.5) (size 0.7) (drill 0.4) (layers F.Cu B.Cu) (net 1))
 (via (at 117 106.5) (size 0.7) (drill 0.4) (layers F.Cu B.Cu) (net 1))
 (via (at 117 105.5) (size 0.7) (drill 0.4) (layers F.Cu B.Cu) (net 1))
 (via (at 117 104.5) (size 0.7) (drill 0.4) (layers F.Cu B.Cu) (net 1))
 (via (at 113 106.5) (size 0.7) (drill 0.4) (layers F.Cu B.Cu) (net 1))
 (via (at 113 105.5) (size 0.7) (drill 0.4) (layers F.Cu B.Cu) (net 1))
 (via (at 113 104.5) (size 0.7) (drill 0.4) (layers F.Cu B.Cu) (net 1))
 (via (at 113 103.5) (size 0.7) (drill 0.4) (layers F.Cu B.Cu) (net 1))
 (via (at 114 103.5) (size 0.7) (drill 0.4) (layers F.Cu B.Cu) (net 1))
 (via (at 115 103.5) (size 0.7) (drill 0.4) (layers F.Cu B.Cu) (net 1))
 (via (at 116 103.5) (size 0.7) (drill 0.4) (layers F.Cu B.Cu) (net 1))
 (via (at 117 103.5) (size 0.7) (drill 0.4) (layers F.Cu B.Cu) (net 1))
 (segment (start 108.875 109) (end 113.429999 109) (width 1.5) (layer F.Cu) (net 4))
 (segment (start 102.032 109) (end 107.05499 109) (width 1.5) (layer F.Cu) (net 2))
 (segment (start 120 107.25) (end 120 105.5) (width 0.22) (layer F.Cu) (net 5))
 (segment (start 120 105.5) (end 120 104) (width 0.22) (layer F.Cu) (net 5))
 (segment (start 120 104) (end 120 101) (width 0.22) (layer F.Cu) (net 5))
 (segment (start 120 109) (end 123.42999 109) (width 1.5) (layer F.Cu) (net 6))
 (segment (start 120 109) (end 116.570001 109) (width 1.5) (layer F.Cu) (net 6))
 (segment (start 130 109) (end 125.25 109) (width 1.5) (layer F.Cu) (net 3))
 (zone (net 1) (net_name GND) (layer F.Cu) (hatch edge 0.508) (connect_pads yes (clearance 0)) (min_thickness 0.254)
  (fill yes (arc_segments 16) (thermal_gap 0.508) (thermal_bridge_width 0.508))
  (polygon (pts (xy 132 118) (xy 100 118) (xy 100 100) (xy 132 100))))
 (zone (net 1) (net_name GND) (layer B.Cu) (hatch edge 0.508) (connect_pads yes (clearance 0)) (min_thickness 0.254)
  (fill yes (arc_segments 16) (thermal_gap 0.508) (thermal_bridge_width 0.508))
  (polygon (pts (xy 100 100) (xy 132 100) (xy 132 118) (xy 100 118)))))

